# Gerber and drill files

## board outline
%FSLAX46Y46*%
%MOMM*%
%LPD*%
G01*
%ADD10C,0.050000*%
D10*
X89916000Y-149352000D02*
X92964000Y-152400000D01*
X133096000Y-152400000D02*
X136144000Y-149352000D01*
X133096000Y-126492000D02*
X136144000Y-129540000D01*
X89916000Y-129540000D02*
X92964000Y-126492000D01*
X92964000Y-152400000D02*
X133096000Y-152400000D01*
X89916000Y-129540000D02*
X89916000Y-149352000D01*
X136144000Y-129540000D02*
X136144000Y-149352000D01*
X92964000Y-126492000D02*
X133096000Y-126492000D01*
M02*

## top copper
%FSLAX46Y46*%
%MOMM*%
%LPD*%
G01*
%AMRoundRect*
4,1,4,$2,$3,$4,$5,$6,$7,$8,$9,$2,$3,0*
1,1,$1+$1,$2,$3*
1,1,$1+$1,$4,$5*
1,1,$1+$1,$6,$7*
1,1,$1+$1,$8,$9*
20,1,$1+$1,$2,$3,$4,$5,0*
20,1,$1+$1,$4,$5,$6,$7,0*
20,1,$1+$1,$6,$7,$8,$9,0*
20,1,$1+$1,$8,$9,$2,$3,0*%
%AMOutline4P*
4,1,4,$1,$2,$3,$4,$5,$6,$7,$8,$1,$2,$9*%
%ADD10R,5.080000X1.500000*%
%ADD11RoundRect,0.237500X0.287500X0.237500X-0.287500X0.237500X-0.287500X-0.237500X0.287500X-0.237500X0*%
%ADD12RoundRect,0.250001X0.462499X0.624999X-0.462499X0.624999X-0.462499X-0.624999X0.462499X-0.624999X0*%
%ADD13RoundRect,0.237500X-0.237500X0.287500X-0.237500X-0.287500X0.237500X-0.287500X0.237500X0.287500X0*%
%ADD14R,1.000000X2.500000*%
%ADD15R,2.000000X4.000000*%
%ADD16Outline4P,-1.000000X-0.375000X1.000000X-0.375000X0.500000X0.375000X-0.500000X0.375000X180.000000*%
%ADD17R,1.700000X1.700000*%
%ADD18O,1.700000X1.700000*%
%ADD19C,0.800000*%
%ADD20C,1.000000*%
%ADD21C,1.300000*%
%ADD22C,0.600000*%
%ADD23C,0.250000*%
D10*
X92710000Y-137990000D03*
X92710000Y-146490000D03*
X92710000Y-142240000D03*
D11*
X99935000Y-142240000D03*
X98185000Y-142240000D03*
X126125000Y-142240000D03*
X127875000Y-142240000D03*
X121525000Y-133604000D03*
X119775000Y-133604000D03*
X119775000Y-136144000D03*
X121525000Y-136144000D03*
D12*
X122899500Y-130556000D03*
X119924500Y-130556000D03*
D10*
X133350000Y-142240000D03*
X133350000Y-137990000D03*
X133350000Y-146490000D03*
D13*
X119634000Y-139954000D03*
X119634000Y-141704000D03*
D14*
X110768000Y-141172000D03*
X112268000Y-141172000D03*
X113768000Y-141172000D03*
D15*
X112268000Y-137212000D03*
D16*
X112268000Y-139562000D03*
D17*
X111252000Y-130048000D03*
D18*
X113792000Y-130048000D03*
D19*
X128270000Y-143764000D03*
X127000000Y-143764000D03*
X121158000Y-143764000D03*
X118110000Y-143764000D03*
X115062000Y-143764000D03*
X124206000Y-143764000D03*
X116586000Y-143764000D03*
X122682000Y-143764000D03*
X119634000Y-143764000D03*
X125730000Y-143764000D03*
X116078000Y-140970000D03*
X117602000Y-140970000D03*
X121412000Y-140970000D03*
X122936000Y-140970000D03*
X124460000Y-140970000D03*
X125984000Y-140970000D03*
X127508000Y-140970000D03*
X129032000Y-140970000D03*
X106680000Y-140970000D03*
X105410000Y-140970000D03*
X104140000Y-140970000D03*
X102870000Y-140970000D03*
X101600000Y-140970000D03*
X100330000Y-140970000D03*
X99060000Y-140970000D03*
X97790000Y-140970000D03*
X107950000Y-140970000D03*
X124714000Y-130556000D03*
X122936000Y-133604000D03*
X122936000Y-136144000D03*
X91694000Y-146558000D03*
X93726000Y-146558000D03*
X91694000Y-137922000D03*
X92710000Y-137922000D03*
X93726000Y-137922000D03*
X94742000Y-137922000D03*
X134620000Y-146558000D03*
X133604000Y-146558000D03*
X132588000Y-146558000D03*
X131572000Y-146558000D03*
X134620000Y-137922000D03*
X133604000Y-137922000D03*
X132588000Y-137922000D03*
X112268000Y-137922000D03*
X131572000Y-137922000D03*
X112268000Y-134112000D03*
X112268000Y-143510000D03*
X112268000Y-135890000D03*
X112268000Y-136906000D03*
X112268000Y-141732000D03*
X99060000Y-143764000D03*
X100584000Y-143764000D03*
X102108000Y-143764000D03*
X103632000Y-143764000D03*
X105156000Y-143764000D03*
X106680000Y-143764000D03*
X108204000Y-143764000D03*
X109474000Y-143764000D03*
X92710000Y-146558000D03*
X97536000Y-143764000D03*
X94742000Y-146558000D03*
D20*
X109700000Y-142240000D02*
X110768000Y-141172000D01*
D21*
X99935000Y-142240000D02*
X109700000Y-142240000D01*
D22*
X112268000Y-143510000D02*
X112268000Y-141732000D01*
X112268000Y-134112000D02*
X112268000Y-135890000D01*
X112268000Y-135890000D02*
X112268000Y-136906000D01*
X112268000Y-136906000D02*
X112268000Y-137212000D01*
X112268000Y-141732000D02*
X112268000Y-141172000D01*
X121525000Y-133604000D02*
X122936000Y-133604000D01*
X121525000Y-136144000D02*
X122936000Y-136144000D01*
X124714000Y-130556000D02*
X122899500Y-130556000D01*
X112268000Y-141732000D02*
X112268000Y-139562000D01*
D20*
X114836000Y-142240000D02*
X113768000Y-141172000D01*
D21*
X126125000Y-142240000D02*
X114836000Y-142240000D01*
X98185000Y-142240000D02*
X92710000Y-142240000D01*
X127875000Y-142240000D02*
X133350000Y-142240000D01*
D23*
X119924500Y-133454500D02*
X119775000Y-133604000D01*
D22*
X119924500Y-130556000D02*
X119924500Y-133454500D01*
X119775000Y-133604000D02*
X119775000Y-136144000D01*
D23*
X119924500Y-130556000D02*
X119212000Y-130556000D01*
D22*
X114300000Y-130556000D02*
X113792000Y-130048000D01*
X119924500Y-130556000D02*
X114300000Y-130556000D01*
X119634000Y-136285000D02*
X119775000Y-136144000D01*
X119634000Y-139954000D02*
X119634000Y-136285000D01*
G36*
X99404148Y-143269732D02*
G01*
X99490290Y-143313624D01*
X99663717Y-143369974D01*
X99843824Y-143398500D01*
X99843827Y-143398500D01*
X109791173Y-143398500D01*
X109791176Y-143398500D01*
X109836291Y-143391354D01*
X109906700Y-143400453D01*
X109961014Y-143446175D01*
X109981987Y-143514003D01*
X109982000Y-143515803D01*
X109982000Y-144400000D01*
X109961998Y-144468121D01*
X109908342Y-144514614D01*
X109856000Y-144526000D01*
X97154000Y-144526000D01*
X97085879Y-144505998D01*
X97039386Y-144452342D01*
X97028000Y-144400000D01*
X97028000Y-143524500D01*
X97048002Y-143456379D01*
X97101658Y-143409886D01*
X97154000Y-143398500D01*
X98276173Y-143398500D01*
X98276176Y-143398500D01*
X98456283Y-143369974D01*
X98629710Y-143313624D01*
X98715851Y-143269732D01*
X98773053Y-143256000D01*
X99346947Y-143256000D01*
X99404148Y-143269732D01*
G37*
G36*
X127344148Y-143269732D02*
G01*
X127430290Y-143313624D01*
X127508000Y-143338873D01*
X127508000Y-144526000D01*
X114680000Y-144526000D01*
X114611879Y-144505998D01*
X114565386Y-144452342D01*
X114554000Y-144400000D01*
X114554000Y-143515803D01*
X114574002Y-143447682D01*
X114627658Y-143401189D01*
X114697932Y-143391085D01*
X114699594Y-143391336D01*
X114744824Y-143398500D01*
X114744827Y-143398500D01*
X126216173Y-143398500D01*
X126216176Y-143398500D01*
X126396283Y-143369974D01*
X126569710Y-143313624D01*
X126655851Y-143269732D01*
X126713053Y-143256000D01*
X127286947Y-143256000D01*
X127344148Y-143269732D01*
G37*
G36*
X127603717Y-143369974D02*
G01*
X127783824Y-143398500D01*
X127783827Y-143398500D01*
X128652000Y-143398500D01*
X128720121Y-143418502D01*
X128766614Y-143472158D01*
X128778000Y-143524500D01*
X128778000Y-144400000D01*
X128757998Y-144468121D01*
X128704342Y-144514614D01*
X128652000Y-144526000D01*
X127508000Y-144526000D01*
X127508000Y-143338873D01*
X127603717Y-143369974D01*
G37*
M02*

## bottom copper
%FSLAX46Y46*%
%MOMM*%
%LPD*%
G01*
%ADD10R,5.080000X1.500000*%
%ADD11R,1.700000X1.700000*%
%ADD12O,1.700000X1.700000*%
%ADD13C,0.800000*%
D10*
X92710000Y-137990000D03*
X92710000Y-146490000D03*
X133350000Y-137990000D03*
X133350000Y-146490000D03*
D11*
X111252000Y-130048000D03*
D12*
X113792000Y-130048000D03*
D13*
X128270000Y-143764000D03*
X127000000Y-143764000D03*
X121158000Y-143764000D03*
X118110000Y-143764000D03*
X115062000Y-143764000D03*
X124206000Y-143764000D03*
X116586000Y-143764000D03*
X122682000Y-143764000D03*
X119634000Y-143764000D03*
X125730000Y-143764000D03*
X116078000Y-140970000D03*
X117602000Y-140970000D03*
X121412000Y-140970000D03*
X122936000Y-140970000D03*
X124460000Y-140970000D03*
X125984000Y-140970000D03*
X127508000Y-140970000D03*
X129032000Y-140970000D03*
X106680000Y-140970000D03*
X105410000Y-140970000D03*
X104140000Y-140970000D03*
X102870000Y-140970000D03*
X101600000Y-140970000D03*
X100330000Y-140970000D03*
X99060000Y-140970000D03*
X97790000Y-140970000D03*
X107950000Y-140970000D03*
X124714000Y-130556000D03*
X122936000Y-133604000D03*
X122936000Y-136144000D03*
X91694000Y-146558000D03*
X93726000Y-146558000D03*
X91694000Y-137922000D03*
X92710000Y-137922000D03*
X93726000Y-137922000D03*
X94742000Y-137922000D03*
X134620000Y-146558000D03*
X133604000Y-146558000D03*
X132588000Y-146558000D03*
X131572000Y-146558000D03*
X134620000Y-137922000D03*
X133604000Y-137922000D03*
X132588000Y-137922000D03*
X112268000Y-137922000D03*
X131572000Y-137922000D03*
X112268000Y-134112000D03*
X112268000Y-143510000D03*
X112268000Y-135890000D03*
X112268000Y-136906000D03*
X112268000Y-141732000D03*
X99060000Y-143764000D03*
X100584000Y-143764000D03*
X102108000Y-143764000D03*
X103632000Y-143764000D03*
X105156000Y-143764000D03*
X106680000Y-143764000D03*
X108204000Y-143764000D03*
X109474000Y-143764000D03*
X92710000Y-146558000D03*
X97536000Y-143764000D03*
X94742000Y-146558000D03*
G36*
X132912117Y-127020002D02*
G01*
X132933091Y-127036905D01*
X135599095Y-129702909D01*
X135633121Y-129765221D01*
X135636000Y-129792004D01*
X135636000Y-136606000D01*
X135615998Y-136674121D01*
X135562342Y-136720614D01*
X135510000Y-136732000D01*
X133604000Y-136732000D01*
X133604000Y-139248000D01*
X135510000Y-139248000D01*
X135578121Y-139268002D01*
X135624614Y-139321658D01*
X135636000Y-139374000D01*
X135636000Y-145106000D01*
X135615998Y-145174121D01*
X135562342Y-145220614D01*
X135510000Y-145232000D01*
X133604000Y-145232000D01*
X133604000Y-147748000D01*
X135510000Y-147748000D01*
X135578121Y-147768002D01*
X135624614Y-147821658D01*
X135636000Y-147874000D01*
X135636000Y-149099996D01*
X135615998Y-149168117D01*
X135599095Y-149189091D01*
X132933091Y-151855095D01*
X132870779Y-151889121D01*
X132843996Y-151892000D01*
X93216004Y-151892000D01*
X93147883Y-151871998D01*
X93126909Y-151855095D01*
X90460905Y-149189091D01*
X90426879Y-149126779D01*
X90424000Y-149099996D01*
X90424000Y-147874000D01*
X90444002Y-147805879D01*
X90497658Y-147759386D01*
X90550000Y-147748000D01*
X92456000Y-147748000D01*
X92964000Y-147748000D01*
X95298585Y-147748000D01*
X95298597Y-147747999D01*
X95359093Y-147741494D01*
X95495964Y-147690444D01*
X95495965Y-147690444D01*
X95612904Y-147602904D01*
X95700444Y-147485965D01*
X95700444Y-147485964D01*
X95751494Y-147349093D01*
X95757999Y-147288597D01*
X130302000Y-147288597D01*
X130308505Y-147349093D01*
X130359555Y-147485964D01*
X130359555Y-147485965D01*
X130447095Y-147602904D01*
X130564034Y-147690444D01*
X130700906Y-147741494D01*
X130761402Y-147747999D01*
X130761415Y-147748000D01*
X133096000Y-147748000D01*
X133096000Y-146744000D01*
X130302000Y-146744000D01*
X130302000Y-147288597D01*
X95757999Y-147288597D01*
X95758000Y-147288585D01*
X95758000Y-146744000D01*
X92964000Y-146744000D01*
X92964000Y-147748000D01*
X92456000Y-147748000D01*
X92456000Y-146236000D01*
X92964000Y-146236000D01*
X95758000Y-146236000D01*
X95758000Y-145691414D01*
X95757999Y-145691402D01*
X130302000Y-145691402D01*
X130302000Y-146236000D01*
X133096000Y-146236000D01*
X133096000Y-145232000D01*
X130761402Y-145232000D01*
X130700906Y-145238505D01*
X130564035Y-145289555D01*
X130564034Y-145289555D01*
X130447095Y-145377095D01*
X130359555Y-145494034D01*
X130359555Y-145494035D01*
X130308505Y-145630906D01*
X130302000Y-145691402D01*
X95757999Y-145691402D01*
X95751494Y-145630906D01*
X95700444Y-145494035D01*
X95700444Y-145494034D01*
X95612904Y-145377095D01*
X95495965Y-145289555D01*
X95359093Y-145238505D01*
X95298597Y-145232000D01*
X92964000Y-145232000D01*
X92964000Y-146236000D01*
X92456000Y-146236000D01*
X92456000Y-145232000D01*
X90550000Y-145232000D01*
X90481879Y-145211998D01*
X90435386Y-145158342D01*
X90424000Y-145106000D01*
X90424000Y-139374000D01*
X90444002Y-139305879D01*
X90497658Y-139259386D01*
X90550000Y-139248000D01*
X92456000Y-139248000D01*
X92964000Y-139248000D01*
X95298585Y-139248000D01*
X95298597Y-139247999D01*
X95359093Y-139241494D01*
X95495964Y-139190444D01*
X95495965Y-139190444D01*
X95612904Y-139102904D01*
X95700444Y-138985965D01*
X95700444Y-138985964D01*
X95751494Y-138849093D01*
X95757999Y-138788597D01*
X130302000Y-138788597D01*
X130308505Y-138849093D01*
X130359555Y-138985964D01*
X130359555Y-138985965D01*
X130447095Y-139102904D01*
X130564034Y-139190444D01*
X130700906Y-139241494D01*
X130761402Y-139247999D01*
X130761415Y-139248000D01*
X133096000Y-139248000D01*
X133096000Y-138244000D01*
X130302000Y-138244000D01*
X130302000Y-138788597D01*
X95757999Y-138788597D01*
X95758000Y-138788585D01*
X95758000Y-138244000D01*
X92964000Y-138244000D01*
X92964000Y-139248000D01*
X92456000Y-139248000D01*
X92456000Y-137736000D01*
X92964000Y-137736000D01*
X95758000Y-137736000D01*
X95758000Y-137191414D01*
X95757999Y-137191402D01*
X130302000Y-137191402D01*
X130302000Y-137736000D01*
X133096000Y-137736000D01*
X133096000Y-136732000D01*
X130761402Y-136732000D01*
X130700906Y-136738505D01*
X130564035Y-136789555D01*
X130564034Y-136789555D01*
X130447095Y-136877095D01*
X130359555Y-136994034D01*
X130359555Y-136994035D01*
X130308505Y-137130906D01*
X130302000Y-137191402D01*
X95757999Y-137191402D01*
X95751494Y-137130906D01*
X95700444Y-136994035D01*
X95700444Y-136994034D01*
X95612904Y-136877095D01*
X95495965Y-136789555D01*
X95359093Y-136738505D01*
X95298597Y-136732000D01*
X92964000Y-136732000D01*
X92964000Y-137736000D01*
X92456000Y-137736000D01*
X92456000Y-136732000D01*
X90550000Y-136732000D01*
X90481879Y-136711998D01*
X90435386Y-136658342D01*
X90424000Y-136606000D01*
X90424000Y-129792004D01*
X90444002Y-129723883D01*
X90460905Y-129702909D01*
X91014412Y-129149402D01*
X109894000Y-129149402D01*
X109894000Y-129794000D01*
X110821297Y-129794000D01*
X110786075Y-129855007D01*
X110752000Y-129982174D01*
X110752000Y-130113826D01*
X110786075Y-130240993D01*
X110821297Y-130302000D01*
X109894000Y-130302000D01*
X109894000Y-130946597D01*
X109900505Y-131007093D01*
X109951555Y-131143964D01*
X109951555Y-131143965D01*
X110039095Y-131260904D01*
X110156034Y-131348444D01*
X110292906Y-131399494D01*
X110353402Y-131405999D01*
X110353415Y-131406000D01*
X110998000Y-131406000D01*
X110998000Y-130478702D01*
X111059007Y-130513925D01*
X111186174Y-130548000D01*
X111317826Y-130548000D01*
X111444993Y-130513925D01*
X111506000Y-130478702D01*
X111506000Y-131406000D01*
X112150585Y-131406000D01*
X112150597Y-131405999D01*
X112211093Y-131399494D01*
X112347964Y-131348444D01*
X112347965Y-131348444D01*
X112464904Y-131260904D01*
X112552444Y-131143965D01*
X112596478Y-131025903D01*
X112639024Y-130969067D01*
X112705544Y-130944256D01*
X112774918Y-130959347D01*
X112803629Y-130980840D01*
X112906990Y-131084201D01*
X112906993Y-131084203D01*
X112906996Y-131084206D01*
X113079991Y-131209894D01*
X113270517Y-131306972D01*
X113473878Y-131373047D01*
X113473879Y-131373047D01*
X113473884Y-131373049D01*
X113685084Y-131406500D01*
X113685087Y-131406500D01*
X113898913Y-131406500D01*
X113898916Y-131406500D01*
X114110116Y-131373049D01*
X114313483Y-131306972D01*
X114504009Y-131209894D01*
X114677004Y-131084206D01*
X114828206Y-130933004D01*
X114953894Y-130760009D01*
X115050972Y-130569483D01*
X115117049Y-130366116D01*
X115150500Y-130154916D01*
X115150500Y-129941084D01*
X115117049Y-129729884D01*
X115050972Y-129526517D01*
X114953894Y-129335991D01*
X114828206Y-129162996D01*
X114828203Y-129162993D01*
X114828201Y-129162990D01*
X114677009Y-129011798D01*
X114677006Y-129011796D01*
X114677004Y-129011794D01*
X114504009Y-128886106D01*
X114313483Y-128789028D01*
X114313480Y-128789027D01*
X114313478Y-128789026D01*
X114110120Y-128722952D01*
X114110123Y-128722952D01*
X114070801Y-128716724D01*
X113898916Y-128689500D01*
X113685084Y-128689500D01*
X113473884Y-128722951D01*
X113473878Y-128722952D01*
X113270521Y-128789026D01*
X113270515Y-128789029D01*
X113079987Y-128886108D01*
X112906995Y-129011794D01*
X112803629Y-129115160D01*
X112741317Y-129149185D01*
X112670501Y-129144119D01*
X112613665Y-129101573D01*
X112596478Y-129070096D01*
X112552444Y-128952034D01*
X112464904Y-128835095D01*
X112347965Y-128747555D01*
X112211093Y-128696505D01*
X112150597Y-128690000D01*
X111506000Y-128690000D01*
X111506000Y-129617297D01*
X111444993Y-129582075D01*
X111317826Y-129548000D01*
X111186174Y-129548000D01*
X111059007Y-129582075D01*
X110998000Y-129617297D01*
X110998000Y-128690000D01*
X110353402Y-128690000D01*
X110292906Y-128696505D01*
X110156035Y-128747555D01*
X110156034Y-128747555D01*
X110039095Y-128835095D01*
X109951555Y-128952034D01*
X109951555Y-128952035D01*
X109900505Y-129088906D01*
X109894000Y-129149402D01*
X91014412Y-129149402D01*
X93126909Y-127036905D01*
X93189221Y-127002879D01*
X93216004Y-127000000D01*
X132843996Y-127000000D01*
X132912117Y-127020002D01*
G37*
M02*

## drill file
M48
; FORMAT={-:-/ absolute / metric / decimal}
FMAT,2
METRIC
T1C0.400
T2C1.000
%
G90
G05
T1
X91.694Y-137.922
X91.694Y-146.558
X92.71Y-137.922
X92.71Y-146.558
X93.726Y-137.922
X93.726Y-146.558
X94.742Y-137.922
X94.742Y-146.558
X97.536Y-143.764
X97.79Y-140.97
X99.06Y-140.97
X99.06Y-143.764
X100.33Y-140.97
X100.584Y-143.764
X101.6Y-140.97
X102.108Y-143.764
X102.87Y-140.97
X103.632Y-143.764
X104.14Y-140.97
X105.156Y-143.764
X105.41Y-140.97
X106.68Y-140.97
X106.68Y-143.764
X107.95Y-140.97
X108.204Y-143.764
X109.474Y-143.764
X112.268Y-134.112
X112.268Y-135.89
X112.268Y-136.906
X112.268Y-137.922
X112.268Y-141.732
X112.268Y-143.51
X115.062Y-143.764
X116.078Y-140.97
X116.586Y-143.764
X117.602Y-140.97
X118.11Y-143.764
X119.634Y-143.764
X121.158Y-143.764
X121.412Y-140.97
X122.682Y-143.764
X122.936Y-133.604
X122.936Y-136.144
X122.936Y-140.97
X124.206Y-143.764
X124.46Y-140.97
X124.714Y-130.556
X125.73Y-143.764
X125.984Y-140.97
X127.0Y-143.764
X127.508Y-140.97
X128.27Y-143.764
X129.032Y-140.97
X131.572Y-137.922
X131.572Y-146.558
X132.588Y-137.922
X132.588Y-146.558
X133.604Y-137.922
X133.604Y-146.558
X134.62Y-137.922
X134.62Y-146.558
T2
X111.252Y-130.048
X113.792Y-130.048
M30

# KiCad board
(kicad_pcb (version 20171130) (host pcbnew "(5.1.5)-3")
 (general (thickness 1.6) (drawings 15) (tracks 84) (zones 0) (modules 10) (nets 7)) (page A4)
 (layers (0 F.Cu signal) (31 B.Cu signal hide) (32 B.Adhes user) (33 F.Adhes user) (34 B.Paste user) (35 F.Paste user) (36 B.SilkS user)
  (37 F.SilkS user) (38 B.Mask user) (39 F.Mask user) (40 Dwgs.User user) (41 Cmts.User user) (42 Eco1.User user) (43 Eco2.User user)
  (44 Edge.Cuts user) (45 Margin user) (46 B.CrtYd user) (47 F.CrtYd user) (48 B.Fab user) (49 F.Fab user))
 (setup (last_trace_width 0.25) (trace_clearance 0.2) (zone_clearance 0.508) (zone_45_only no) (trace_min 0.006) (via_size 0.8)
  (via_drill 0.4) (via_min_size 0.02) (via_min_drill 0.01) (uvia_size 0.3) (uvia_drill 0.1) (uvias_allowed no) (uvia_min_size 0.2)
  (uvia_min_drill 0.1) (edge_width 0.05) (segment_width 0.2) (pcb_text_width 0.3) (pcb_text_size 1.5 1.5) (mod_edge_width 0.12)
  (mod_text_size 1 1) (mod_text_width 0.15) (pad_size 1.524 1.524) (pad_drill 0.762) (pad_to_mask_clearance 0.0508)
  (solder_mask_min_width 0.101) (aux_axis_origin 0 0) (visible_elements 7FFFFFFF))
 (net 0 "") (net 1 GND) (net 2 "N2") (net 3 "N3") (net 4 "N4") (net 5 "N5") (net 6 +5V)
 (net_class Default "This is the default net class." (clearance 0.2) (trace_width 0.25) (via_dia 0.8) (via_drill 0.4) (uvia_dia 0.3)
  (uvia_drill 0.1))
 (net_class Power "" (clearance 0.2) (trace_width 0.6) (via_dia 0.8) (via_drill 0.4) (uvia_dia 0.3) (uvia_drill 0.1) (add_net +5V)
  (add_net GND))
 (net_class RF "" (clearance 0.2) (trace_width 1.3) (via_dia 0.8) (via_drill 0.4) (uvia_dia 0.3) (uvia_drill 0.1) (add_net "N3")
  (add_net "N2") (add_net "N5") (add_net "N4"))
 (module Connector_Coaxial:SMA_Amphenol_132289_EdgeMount (layer F.Cu) (at 92.71 142.24 180)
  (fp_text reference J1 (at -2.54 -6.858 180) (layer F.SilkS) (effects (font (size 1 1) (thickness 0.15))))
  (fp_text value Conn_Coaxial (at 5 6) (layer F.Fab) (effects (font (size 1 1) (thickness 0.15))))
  (pad 2 smd rect (at 0 4.25 270) (size 1.5 5.08) (layers B.Cu B.Paste B.Mask) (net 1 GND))
  (pad 2 smd rect (at 0 -4.25 270) (size 1.5 5.08) (layers B.Cu B.Paste B.Mask) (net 1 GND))
  (pad 2 smd rect (at 0 4.25 270) (size 1.5 5.08) (layers F.Cu F.Paste F.Mask) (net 1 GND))
  (pad 2 smd rect (at 0 -4.25 270) (size 1.5 5.08) (layers F.Cu F.Paste F.Mask) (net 1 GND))
  (pad 1 smd rect (at 0 0 270) (size 1.5 5.08) (layers F.Cu F.Paste F.Mask) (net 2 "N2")))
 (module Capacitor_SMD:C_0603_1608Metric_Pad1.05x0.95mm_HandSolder (layer F.Cu) (at 99.06 142.24 180)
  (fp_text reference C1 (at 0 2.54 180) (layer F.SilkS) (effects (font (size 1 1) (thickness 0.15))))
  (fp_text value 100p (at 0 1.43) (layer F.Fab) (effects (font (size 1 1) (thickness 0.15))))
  (pad 1 smd roundrect (at -0.875 0 180) (size 1.05 0.95) (layers F.Cu F.Paste F.Mask) (roundrect_rratio 0.25) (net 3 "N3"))
  (pad 2 smd roundrect (at 0.875 0 180) (size 1.05 0.95) (layers F.Cu F.Paste F.Mask) (roundrect_rratio 0.25) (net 2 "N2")))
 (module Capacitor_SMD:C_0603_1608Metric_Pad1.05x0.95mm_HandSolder (layer F.Cu) (at 127 142.24 180)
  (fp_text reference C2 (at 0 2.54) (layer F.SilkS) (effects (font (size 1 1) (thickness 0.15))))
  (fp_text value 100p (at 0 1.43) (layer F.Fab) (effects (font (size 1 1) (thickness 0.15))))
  (pad 2 smd roundrect (at 0.875 0 180) (size 1.05 0.95) (layers F.Cu F.Paste F.Mask) (roundrect_rratio 0.25) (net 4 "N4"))
  (pad 1 smd roundrect (at -0.875 0 180) (size 1.05 0.95) (layers F.Cu F.Paste F.Mask) (roundrect_rratio 0.25) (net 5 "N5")))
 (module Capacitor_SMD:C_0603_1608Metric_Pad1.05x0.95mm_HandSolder (layer F.Cu) (at 120.65 133.604 180)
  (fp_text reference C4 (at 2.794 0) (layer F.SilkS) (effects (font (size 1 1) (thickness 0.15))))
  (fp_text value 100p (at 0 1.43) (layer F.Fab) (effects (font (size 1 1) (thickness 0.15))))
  (pad 1 smd roundrect (at -0.875 0 180) (size 1.05 0.95) (layers F.Cu F.Paste F.Mask) (roundrect_rratio 0.25) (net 1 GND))
  (pad 2 smd roundrect (at 0.875 0 180) (size 1.05 0.95) (layers F.Cu F.Paste F.Mask) (roundrect_rratio 0.25) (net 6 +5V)))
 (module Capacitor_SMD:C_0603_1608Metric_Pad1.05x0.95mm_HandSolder (layer F.Cu) (at 120.65 136.144 180)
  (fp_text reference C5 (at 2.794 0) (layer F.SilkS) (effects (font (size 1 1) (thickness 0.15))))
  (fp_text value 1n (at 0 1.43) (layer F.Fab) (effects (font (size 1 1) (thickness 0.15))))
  (pad 2 smd roundrect (at 0.875 0 180) (size 1.05 0.95) (layers F.Cu F.Paste F.Mask) (roundrect_rratio 0.25) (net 6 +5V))
  (pad 1 smd roundrect (at -0.875 0 180) (size 1.05 0.95) (layers F.Cu F.Paste F.Mask) (roundrect_rratio 0.25) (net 1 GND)))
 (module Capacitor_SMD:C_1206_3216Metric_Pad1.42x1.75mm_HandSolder (layer F.Cu) (at 121.412 130.556 180)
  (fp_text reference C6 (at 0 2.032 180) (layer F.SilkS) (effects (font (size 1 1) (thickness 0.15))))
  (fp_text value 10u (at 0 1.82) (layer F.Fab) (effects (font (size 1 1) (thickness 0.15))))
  (pad 1 smd roundrect (at -1.4875 0 180) (size 1.425 1.75) (layers F.Cu F.Paste F.Mask) (roundrect_rratio 0.175439) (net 1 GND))
  (pad 2 smd roundrect (at 1.4875 0 180) (size 1.425 1.75) (layers F.Cu F.Paste F.Mask) (roundrect_rratio 0.175439) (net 6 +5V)))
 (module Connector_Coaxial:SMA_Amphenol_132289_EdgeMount (layer F.Cu) (at 133.35 142.24)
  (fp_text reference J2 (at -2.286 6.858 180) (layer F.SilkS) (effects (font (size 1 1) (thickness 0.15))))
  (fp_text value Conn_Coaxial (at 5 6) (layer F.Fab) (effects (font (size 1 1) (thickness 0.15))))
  (pad 1 smd rect (at 0 0 90) (size 1.5 5.08) (layers F.Cu F.Paste F.Mask) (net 5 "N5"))
  (pad 2 smd rect (at 0 -4.25 90) (size 1.5 5.08) (layers F.Cu F.Paste F.Mask) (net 1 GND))
  (pad 2 smd rect (at 0 4.25 90) (size 1.5 5.08) (layers F.Cu F.Paste F.Mask) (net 1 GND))
  (pad 2 smd rect (at 0 -4.25 90) (size 1.5 5.08) (layers B.Cu B.Paste B.Mask) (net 1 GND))
  (pad 2 smd rect (at 0 4.25 90) (size 1.5 5.08) (layers B.Cu B.Paste B.Mask) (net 1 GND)))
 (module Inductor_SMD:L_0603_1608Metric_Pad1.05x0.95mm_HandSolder (layer F.Cu) (at 119.634 140.829 270)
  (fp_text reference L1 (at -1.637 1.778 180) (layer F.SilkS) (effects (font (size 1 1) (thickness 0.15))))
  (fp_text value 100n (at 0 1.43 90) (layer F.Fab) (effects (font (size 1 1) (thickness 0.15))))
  (pad 1 smd roundrect (at -0.875 0 270) (size 1.05 0.95) (layers F.Cu F.Paste F.Mask) (roundrect_rratio 0.25) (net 6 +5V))
  (pad 2 smd roundrect (at 0.875 0 270) (size 1.05 0.95) (layers F.Cu F.Paste F.Mask) (roundrect_rratio 0.25) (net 4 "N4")))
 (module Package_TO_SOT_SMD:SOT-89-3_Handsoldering (layer F.Cu) (at 112.268 139.192 90)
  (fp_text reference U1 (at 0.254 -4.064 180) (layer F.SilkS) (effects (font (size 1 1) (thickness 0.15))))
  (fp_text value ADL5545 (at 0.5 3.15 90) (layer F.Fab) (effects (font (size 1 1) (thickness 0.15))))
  (pad 1 smd rect (at -1.98 -1.5) (size 1 2.5) (layers F.Cu F.Paste F.Mask) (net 3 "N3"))
  (pad 2 smd rect (at -1.98 0) (size 1 2.5) (layers F.Cu F.Paste F.Mask) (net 1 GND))
  (pad 3 smd rect (at -1.98 1.5) (size 1 2.5) (layers F.Cu F.Paste F.Mask) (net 4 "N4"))
  (pad 2 smd rect (at 1.98 0) (size 2 4) (layers F.Cu F.Paste F.Mask) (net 1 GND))
  (pad 2 smd trapezoid (at -0.37 0 180) (size 1.5 0.75) (rect_delta 0 0.5) (layers F.Cu F.Paste F.Mask) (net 1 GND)))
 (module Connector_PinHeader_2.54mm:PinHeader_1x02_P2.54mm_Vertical (layer F.Cu) (at 111.252 130.048 90)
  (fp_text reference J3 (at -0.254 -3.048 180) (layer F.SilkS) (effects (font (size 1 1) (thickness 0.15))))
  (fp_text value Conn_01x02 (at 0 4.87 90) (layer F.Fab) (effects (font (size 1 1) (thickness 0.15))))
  (pad 1 thru_hole rect (at 0 0 90) (size 1.7 1.7) (drill 1) (layers *.Cu *.Mask) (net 1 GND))
  (pad 2 thru_hole oval (at 0 2.54 90) (size 1.7 1.7) (drill 1) (layers *.Cu *.Mask) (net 6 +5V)))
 (gr_line (start 89.916 149.352) (end 92.964 152.4) (layer Edge.Cuts) (width 0.05))
 (gr_line (start 133.096 152.4) (end 136.144 149.352) (layer Edge.Cuts) (width 0.05))
 (gr_line (start 133.096 126.492) (end 136.144 129.54) (layer Edge.Cuts) (width 0.05))
 (gr_line (start 89.916 129.54) (end 92.964 126.492) (layer Edge.Cuts) (width 0.05))
 (gr_line (start 92.964 152.4) (end 133.096 152.4) (layer Edge.Cuts) (width 0.05))
 (gr_line (start 89.916 129.54) (end 89.916 149.352) (layer Edge.Cuts) (width 0.05))
 (gr_line (start 136.144 129.54) (end 136.144 149.352) (layer Edge.Cuts) (width 0.05))
 (gr_line (start 92.964 126.492) (end 133.096 126.492) (layer Edge.Cuts) (width 0.05))
 (segment (start 109.7 142.24) (end 110.768 141.172) (width 1) (layer F.Cu) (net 3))
 (segment (start 99.935 142.24) (end 109.7 142.24) (width 1.3) (layer F.Cu) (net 3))
 (via (at 128.27 143.764) (size 0.8) (drill 0.4) (layers F.Cu B.Cu) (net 1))
 (via (at 127 143.764) (size 0.8) (drill 0.4) (layers F.Cu B.Cu) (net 1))
 (via (at 121.158 143.764) (size 0.8) (drill 0.4) (layers F.Cu B.Cu) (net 1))
 (via (at 118.11 143.764) (size 0.8) (drill 0.4) (layers F.Cu B.Cu) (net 1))
 (via (at 115.062 143.764) (size 0.8) (drill 0.4) (layers F.Cu B.Cu) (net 1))
 (via (at 124.206 143.764) (size 0.8) (drill 0.4) (layers F.Cu B.Cu) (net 1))
 (via (at 116.586 143.764) (size 0.8) (drill 0.4) (layers F.Cu B.Cu) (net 1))
 (via (at 122.682 143.764) (size 0.8) (drill 0.4) (layers F.Cu B.Cu) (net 1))
 (via (at 119.634 143.764) (size 0.8) (drill 0.4) (layers F.Cu B.Cu) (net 1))
 (via (at 125.73 143.764) (size 0.8) (drill 0.4) (layers F.Cu B.Cu) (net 1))
 (via (at 116.078 140.97) (size 0.8) (drill 0.4) (layers F.Cu B.Cu) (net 1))
 (via (at 117.602 140.97) (size 0.8) (drill 0.4) (layers F.Cu B.Cu) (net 1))
 (via (at 121.412 140.97) (size 0.8) (drill 0.4) (layers F.Cu B.Cu) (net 1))
 (via (at 122.936 140.97) (size 0.8) (drill 0.4) (layers F.Cu B.Cu) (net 1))
 (via (at 124.46 140.97) (size 0.8) (drill 0.4) (layers F.Cu B.Cu) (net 1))
 (via (at 125.984 140.97) (size 0.8) (drill 0.4) (layers F.Cu B.Cu) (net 1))
 (via (at 127.508 140.97) (size 0.8) (drill 0.4) (layers F.Cu B.Cu) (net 1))
 (via (at 129.032 140.97) (size 0.8) (drill 0.4) (layers F.Cu B.Cu) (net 1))
 (via (at 106.68 140.97) (size 0.8) (drill 0.4) (layers F.Cu B.Cu) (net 1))
 (via (at 105.41 140.97) (size 0.8) (drill 0.4) (layers F.Cu B.Cu) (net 1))
 (via (at 104.14 140.97) (size 0.8) (drill 0.4) (layers F.Cu B.Cu) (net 1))
 (via (at 102.87 140.97) (size 0.8) (drill 0.4) (layers F.Cu B.Cu) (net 1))
 (via (at 101.6 140.97) (size 0.8) (drill 0.4) (layers F.Cu B.Cu) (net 1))
 (via (at 100.33 140.97) (size 0.8) (drill 0.4) (layers F.Cu B.Cu) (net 1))
 (via (at 99.06 140.97) (size 0.8) (drill 0.4) (layers F.Cu B.Cu) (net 1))
 (via (at 97.79 140.97) (size 0.8) (drill 0.4) (layers F.Cu B.Cu) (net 1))
 (via (at 107.95 140.97) (size 0.8) (drill 0.4) (layers F.Cu B.Cu) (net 1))
 (via (at 124.714 130.556) (size 0.8) (drill 0.4) (layers F.Cu B.Cu) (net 1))
 (via (at 122.936 133.604) (size 0.8) (drill 0.4) (layers F.Cu B.Cu) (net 1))
 (via (at 122.936 136.144) (size 0.8) (drill 0.4) (layers F.Cu B.Cu) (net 1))
 (via (at 91.694 146.558) (size 0.8) (drill 0.4) (layers F.Cu B.Cu) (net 1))
 (via (at 93.726 146.558) (size 0.8) (drill 0.4) (layers F.Cu B.Cu) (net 1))
 (via (at 91.694 137.922) (size 0.8) (drill 0.4) (layers F.Cu B.Cu) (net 1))
 (via (at 92.71 137.922) (size 0.8) (drill 0.4) (layers F.Cu B.Cu) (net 1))
 (via (at 93.726 137.922) (size 0.8) (drill 0.4) (layers F.Cu B.Cu) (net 1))
 (via (at 94.742 137.922) (size 0.8) (drill 0.4) (layers F.Cu B.Cu) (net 1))
 (via (at 134.62 146.558) (size 0.8) (drill 0.4) (layers F.Cu B.Cu) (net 1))
 (via (at 133.604 146.558) (size 0.8) (drill 0.4) (layers F.Cu B.Cu) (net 1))
 (via (at 132.588 146.558) (size 0.8) (drill 0.4) (layers F.Cu B.Cu) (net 1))
 (via (at 131.572 146.558) (size 0.8) (drill 0.4) (layers F.Cu B.Cu) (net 1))
 (via (at 134.62 137.922) (size 0.8) (drill 0.4) (layers F.Cu B.Cu) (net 1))
 (via (at 133.604 137.922) (size 0.8) (drill 0.4) (layers F.Cu B.Cu) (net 1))
 (via (at 132.588 137.922) (size 0.8) (drill 0.4) (layers F.Cu B.Cu) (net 1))
 (via (at 112.268 137.922) (size 0.8) (drill 0.4) (layers F.Cu B.Cu) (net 1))
 (via (at 131.572 137.922) (size 0.8) (drill 0.4) (layers F.Cu B.Cu) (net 1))
 (via (at 112.268 134.112) (size 0.8) (drill 0.4) (layers F.Cu B.Cu) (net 1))
 (via (at 112.268 143.51) (size 0.8) (drill 0.4) (layers F.Cu B.Cu) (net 1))
 (segment (start 112.268 143.51) (end 112.268 141.732) (width 0.6) (layer F.Cu) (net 1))
 (segment (start 112.268 134.112) (end 112.268 135.89) (width 0.6) (layer F.Cu) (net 1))
 (segment (start 112.268 135.89) (end 112.268 136.906) (width 0.6) (layer F.Cu) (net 1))
 (via (at 112.268 135.89) (size 0.8) (drill 0.4) (layers F.Cu B.Cu) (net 1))
 (segment (start 112.268 136.906) (end 112.268 137.212) (width 0.6) (layer F.Cu) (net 1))
 (via (at 112.268 136.906) (size 0.8) (drill 0.4) (layers F.Cu B.Cu) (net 1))
 (segment (start 112.268 141.732) (end 112.268 141.172) (width 0.6) (layer F.Cu) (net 1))
 (via (at 112.268 141.732) (size 0.8) (drill 0.4) (layers F.Cu B.Cu) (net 1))
 (segment (start 121.525 133.604) (end 122.936 133.604) (width 0.6) (layer F.Cu) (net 1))
 (segment (start 121.525 136.144) (end 122.936 136.144) (width 0.6) (layer F.Cu) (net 1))
 (segment (start 124.714 130.556) (end 122.8995 130.556) (width 0.6) (layer F.Cu) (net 1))
 (via (at 99.06 143.764) (size 0.8) (drill 0.4) (layers F.Cu B.Cu) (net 1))
 (via (at 100.584 143.764) (size 0.8) (drill 0.4) (layers F.Cu B.Cu) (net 1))
 (via (at 102.108 143.764) (size 0.8) (drill 0.4) (layers F.Cu B.Cu) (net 1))
 (via (at 103.632 143.764) (size 0.8) (drill 0.4) (layers F.Cu B.Cu) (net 1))
 (via (at 105.156 143.764) (size 0.8) (drill 0.4) (layers F.Cu B.Cu) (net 1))
 (via (at 106.68 143.764) (size 0.8) (drill 0.4) (layers F.Cu B.Cu) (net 1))
 (via (at 108.204 143.764) (size 0.8) (drill 0.4) (layers F.Cu B.Cu) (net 1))
 (via (at 109.474 143.764) (size 0.8) (drill 0.4) (layers F.Cu B.Cu) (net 1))
 (segment (start 112.268 141.732) (end 112.268 139.562) (width 0.6) (layer F.Cu) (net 1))
 (via (at 92.71 146.558) (size 0.8) (drill 0.4) (layers F.Cu B.Cu) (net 1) (status 1000000))
 (via (at 97.536 143.764) (size 0.8) (drill 0.4) (layers F.Cu B.Cu) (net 1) (status 1000000))
 (via (at 94.742 146.558) (size 0.8) (drill 0.4) (layers F.Cu B.Cu) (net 1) (status 1000000))
 (segment (start 114.836 142.24) (end 113.768 141.172) (width 1) (layer F.Cu) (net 4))
 (segment (start 126.125 142.24) (end 114.836 142.24) (width 1.3) (layer F.Cu) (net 4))
 (segment (start 98.185 142.24) (end 92.71 142.24) (width 1.3) (layer F.Cu) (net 2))
 (segment (start 127.875 142.24) (end 133.35 142.24) (width 1.3) (layer F.Cu) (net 5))
 (segment (start 119.9245 133.4545) (end 119.775 133.604) (width 0.25) (layer F.Cu) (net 6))
 (segment (start 119.9245 130.556) (end 119.9245 133.4545) (width 0.6) (layer F.Cu) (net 6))
 (segment (start 119.775 133.604) (end 119.775 136.144) (width 0.6) (layer F.Cu) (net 6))
 (segment (start 119.9245 130.556) (end 119.212 130.556) (width 0.25) (layer F.Cu) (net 6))
 (segment (start 114.3 130.556) (end 113.792 130.048) (width 0.6) (layer F.Cu) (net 6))
 (segment (start 119.9245 130.556) (end 114.3 130.556) (width 0.6) (layer F.Cu) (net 6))
 (segment (start 119.634 136.285) (end 119.775 136.144) (width 0.6) (layer F.Cu) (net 6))
 (segment (start 119.634 139.954) (end 119.634 136.285) (width 0.6) (layer F.Cu) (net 6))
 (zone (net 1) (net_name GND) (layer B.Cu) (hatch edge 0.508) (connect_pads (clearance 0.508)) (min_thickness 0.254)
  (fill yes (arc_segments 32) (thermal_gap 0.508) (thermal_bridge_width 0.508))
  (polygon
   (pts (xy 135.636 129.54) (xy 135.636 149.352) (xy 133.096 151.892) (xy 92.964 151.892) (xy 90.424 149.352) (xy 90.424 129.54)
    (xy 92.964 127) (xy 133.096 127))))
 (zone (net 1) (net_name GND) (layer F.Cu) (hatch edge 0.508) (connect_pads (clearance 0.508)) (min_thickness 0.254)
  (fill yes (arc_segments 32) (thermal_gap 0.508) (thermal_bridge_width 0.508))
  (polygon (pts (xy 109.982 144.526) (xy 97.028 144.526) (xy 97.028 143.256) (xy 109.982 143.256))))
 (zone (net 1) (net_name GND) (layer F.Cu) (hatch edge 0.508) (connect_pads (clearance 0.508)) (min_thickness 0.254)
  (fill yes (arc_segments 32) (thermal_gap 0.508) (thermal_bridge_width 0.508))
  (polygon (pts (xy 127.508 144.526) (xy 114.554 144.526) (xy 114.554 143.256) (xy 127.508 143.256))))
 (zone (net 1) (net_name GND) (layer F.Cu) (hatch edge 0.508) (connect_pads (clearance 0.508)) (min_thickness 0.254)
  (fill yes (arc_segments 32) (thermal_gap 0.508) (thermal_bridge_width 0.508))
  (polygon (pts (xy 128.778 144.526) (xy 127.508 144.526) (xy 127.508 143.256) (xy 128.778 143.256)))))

